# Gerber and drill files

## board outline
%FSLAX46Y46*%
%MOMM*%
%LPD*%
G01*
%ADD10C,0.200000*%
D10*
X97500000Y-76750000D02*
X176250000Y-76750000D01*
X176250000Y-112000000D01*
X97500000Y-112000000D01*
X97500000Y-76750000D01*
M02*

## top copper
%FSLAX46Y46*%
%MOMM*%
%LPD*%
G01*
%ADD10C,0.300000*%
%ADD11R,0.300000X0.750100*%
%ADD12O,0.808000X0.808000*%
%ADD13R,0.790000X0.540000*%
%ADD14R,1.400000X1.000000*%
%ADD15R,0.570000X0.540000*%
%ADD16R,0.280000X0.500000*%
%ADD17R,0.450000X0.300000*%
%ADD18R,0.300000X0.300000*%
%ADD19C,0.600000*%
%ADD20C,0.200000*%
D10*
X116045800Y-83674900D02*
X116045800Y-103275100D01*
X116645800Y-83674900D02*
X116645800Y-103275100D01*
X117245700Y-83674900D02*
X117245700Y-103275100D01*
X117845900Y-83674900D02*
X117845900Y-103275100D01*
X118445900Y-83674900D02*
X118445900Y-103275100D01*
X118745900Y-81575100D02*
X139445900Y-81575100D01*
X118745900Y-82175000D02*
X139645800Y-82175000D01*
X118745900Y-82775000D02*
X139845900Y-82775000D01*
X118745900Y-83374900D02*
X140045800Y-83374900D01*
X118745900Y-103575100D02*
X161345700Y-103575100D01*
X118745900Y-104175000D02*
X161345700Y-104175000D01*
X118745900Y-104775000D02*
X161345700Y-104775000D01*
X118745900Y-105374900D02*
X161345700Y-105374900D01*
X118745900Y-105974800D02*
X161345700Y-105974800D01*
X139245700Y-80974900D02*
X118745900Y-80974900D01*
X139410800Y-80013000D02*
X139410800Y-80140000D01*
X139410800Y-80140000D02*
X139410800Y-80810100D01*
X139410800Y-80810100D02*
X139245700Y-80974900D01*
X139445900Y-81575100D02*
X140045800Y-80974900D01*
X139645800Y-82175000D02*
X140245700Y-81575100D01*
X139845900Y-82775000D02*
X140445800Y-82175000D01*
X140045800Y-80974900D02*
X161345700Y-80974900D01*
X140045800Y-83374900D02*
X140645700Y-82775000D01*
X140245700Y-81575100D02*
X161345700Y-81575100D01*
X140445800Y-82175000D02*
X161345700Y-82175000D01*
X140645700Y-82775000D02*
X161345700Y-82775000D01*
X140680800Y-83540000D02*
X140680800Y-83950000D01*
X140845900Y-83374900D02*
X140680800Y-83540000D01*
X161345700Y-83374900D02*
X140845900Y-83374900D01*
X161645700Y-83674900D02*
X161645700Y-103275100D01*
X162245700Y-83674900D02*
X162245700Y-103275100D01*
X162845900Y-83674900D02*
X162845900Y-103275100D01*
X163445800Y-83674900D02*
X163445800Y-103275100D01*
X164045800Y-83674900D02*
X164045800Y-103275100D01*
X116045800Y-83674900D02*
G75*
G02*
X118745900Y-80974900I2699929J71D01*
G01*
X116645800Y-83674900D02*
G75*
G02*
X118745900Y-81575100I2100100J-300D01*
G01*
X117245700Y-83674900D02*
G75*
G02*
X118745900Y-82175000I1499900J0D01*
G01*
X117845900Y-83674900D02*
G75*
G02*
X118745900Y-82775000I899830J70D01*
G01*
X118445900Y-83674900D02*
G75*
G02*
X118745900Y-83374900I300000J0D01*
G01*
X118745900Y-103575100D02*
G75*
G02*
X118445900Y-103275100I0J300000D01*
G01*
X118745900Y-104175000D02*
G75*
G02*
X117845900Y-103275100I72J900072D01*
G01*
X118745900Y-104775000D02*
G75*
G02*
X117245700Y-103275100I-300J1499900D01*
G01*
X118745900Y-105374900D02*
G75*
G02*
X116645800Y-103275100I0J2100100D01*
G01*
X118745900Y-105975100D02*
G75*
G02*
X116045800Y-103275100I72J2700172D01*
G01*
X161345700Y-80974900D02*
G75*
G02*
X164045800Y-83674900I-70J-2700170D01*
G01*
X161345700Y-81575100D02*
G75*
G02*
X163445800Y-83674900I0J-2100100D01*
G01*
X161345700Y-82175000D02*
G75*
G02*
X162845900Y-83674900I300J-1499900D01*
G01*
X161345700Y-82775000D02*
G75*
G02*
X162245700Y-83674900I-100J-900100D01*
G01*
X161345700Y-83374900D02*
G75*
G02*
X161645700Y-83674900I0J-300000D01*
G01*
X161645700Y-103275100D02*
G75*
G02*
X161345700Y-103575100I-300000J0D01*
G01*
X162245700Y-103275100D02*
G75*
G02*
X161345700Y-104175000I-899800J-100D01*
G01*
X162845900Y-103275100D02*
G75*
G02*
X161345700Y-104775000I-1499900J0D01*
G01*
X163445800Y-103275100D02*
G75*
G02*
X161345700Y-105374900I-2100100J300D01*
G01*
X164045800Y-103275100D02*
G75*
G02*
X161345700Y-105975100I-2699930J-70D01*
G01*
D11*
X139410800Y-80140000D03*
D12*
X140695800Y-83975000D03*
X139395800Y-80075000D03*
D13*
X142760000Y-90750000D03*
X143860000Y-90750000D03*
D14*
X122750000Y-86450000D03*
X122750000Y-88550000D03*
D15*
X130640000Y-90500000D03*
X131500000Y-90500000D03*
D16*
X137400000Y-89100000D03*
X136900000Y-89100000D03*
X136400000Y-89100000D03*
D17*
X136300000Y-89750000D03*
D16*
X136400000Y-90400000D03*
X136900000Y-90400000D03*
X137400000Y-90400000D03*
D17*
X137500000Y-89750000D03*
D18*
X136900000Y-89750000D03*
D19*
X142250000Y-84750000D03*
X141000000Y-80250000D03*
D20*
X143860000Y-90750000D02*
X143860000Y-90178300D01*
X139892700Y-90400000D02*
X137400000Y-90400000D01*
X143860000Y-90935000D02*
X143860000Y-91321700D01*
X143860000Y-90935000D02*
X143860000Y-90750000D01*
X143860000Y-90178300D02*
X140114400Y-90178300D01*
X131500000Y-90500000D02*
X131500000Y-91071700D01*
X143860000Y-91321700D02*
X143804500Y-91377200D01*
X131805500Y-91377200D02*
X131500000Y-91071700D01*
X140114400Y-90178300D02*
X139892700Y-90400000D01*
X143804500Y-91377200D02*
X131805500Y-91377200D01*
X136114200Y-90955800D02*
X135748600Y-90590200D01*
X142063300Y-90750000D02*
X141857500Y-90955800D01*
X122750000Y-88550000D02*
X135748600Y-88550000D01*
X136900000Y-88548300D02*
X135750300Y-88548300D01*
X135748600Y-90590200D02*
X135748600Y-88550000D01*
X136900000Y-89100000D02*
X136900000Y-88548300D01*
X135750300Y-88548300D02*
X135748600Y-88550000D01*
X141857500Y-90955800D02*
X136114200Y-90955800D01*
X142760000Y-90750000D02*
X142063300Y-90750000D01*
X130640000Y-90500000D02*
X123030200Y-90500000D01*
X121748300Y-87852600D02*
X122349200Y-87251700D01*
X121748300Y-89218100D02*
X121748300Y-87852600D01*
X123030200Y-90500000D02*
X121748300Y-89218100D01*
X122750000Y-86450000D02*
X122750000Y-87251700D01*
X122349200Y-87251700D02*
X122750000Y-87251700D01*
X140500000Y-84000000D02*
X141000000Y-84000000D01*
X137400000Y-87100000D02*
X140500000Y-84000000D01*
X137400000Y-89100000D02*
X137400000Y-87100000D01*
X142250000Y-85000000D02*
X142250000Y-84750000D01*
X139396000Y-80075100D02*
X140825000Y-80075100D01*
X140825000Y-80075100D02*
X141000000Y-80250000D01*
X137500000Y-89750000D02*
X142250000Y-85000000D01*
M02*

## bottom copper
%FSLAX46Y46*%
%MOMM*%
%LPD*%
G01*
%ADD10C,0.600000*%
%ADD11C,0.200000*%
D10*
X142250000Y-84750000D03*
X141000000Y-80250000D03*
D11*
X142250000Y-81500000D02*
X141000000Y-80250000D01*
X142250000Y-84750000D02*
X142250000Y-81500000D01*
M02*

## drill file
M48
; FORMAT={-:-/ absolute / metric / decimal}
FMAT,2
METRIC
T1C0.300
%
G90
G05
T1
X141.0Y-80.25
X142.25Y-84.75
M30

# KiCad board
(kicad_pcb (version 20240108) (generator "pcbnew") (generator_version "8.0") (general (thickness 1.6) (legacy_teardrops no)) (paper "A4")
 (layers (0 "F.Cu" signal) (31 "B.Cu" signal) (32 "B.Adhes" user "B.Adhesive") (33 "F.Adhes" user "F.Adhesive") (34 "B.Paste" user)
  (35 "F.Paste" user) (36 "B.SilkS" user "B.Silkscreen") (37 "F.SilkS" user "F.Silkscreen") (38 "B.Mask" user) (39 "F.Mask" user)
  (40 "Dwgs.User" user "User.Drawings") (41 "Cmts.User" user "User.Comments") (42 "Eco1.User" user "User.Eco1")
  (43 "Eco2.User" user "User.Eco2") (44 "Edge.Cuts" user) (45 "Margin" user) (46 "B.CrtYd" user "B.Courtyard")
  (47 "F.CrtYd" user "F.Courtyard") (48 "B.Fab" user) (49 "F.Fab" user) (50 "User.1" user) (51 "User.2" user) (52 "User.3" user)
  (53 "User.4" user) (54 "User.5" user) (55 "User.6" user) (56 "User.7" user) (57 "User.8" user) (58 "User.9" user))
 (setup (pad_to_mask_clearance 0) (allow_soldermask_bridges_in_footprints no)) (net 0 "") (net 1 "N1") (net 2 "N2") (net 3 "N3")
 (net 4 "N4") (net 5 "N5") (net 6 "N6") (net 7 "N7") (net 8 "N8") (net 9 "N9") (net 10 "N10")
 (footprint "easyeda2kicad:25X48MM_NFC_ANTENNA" (layer "F.Cu") (at 140.0458 93.475)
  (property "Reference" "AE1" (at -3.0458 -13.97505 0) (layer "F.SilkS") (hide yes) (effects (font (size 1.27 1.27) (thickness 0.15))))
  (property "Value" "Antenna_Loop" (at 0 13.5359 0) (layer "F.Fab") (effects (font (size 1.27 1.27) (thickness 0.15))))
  (fp_line (start -24 -9.8001) (end -24 9.8001) (stroke (width 0.3) (type default)) (layer "F.Cu"))
  (fp_line (start -23.4 -9.8001) (end -23.4 9.8001) (stroke (width 0.3) (type default)) (layer "F.Cu"))
  (fp_line (start -22.8001 -9.8001) (end -22.8001 9.8001) (stroke (width 0.3) (type default)) (layer "F.Cu"))
  (fp_line (start -22.1999 -9.8001) (end -22.1999 9.8001) (stroke (width 0.3) (type default)) (layer "F.Cu"))
  (fp_line (start -21.5999 -9.8001) (end -21.5999 9.8001) (stroke (width 0.3) (type default)) (layer "F.Cu"))
  (fp_line (start -21.2999 -11.8999) (end -0.5999 -11.8999) (stroke (width 0.3) (type default)) (layer "F.Cu"))
  (fp_line (start -21.2999 -11.3) (end -0.4 -11.3) (stroke (width 0.3) (type default)) (layer "F.Cu"))
  (fp_line (start -21.2999 -10.7) (end -0.1999 -10.7) (stroke (width 0.3) (type default)) (layer "F.Cu"))
  (fp_line (start -21.2999 -10.1001) (end 0 -10.1001) (stroke (width 0.3) (type default)) (layer "F.Cu"))
  (fp_line (start -21.2999 10.1001) (end 21.2999 10.1001) (stroke (width 0.3) (type default)) (layer "F.Cu"))
  (fp_line (start -21.2999 10.7) (end 21.2999 10.7) (stroke (width 0.3) (type default)) (layer "F.Cu"))
  (fp_line (start -21.2999 11.3) (end 21.2999 11.3) (stroke (width 0.3) (type default)) (layer "F.Cu"))
  (fp_line (start -21.2999 11.8999) (end 21.2999 11.8999) (stroke (width 0.3) (type default)) (layer "F.Cu"))
  (fp_line (start -21.2999 12.4998) (end 21.2999 12.4998) (stroke (width 0.3) (type default)) (layer "F.Cu"))
  (fp_line (start -0.8001 -12.5001) (end -21.2999 -12.5001) (stroke (width 0.3) (type default)) (layer "F.Cu"))
  (fp_line (start -0.635 -13.462) (end -0.635 -13.335) (stroke (width 0.3) (type default)) (layer "F.Cu"))
  (fp_line (start -0.635 -13.335) (end -0.635 -12.6649) (stroke (width 0.3) (type default)) (layer "F.Cu"))
  (fp_line (start -0.635 -12.6649) (end -0.8001 -12.5001) (stroke (width 0.3) (type default)) (layer "F.Cu"))
  (fp_line (start -0.5999 -11.8999) (end 0 -12.5001) (stroke (width 0.3) (type default)) (layer "F.Cu"))
  (fp_line (start -0.4 -11.3) (end 0.1999 -11.8999) (stroke (width 0.3) (type default)) (layer "F.Cu"))
  (fp_line (start -0.1999 -10.7) (end 0.4 -11.3) (stroke (width 0.3) (type default)) (layer "F.Cu"))
  (fp_line (start 0 -12.5001) (end 21.2999 -12.5001) (stroke (width 0.3) (type default)) (layer "F.Cu"))
  (fp_line (start 0 -10.1001) (end 0.5999 -10.7) (stroke (width 0.3) (type default)) (layer "F.Cu"))
  (fp_line (start 0.1999 -11.8999) (end 21.2999 -11.8999) (stroke (width 0.3) (type default)) (layer "F.Cu"))
  (fp_line (start 0.4 -11.3) (end 21.2999 -11.3) (stroke (width 0.3) (type default)) (layer "F.Cu"))
  (fp_line (start 0.5999 -10.7) (end 21.2999 -10.7) (stroke (width 0.3) (type default)) (layer "F.Cu"))
  (fp_line (start 0.635 -9.935) (end 0.635 -9.525) (stroke (width 0.3) (type default)) (layer "F.Cu"))
  (fp_line (start 0.8001 -10.1001) (end 0.635 -9.935) (stroke (width 0.3) (type default)) (layer "F.Cu"))
  (fp_line (start 21.2999 -10.1001) (end 0.8001 -10.1001) (stroke (width 0.3) (type default)) (layer "F.Cu"))
  (fp_line (start 21.5999 -9.8001) (end 21.5999 9.8001) (stroke (width 0.3) (type default)) (layer "F.Cu"))
  (fp_line (start 22.1999 -9.8001) (end 22.1999 9.8001) (stroke (width 0.3) (type default)) (layer "F.Cu"))
  (fp_line (start 22.8001 -9.8001) (end 22.8001 9.8001) (stroke (width 0.3) (type default)) (layer "F.Cu"))
  (fp_line (start 23.4 -9.8001) (end 23.4 9.8001) (stroke (width 0.3) (type default)) (layer "F.Cu"))
  (fp_line (start 24 -9.8001) (end 24 9.8001) (stroke (width 0.3) (type default)) (layer "F.Cu"))
  (fp_arc (start -24 -9.8001) (mid -23.209174 -11.709344) (end -21.2999 -12.5001) (stroke (width 0.3) (type default)) (layer "F.Cu"))
  (fp_arc (start -23.4 -9.8001) (mid -22.784789 -11.284901) (end -21.2999 -11.8999) (stroke (width 0.3) (type default)) (layer "F.Cu"))
  (fp_arc (start -22.8001 -9.8001) (mid -22.360683 -10.860796) (end -21.2999 -11.3) (stroke (width 0.3) (type default)) (layer "F.Cu"))
  (fp_arc (start -22.1999 -9.8001) (mid -21.936311 -10.436481) (end -21.2999 -10.7) (stroke (width 0.3) (type default)) (layer "F.Cu"))
  (fp_arc (start -21.5999 -9.8001) (mid -21.512032 -10.012232) (end -21.2999 -10.1001) (stroke (width 0.3) (type default)) (layer "F.Cu"))
  (fp_arc (start -21.2999 10.1001) (mid -21.512032 10.012232) (end -21.5999 9.8001) (stroke (width 0.3) (type default)) (layer "F.Cu"))
  (fp_arc (start -21.2999 10.7) (mid -21.93624 10.43641) (end -22.1999 9.8001) (stroke (width 0.3) (type default)) (layer "F.Cu"))
  (fp_arc (start -21.2999 11.3) (mid -22.360683 10.860796) (end -22.8001 9.8001) (stroke (width 0.3) (type default)) (layer "F.Cu"))
  (fp_arc (start -21.2999 11.8999) (mid -22.784789 11.284901) (end -23.4 9.8001) (stroke (width 0.3) (type default)) (layer "F.Cu"))
  (fp_arc (start -21.2999 12.5001) (mid -23.209103 11.709273) (end -24 9.8001) (stroke (width 0.3) (type default)) (layer "F.Cu"))
  (fp_arc (start 21.2999 -12.5001) (mid 23.209103 -11.709274) (end 24 -9.8001) (stroke (width 0.3) (type default)) (layer "F.Cu"))
  (fp_arc (start 21.2999 -11.8999) (mid 22.784789 -11.284901) (end 23.4 -9.8001) (stroke (width 0.3) (type default)) (layer "F.Cu"))
  (fp_arc (start 21.2999 -11.3) (mid 22.360683 -10.860796) (end 22.8001 -9.8001) (stroke (width 0.3) (type default)) (layer "F.Cu"))
  (fp_arc (start 21.2999 -10.7) (mid 21.936231 -10.436402) (end 22.1999 -9.8001) (stroke (width 0.3) (type default)) (layer "F.Cu"))
  (fp_arc (start 21.2999 -10.1001) (mid 21.512032 -10.012232) (end 21.5999 -9.8001) (stroke (width 0.3) (type default)) (layer "F.Cu"))
  (fp_arc (start 21.5999 9.8001) (mid 21.512032 10.012232) (end 21.2999 10.1001) (stroke (width 0.3) (type default)) (layer "F.Cu"))
  (fp_arc (start 22.1999 9.8001) (mid 21.936319 10.43649) (end 21.2999 10.7) (stroke (width 0.3) (type default)) (layer "F.Cu"))
  (fp_arc (start 22.8001 9.8001) (mid 22.360683 10.860796) (end 21.2999 11.3) (stroke (width 0.3) (type default)) (layer "F.Cu"))
  (fp_arc (start 23.4 9.8001) (mid 22.784789 11.284901) (end 21.2999 11.8999) (stroke (width 0.3) (type default)) (layer "F.Cu"))
  (fp_arc (start 24 9.8001) (mid 23.209173 11.709344) (end 21.2999 12.5001) (stroke (width 0.3) (type default)) (layer "F.Cu"))
  (pad "P$1" smd rect (at -0.635 -13.335 90) (size 0.7501 0.3) (layers "F.Cu" "F.Paste" "F.Mask") (solder_mask_margin 0.1016)
   (thermal_bridge_angle 0))
  (pad "P$2" smd oval (at 0.65 -9.5) (size 0.808 0.808) (layers "F.Cu" "F.Paste" "F.Mask") (solder_mask_margin 0.1016)
   (thermal_bridge_angle 0))
  (pad "P$4" smd oval (at -0.65 -13.4) (size 0.808 0.808) (layers "F.Cu" "F.Paste" "F.Mask") (solder_mask_margin 0.1016)
   (thermal_bridge_angle 0)))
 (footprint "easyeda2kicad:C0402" (layer "F.Cu") (at 143.31 90.75)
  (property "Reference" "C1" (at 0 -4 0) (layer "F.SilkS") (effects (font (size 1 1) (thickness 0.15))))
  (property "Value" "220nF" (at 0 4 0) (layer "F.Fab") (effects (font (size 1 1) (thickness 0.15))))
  (pad "1" smd rect (at -0.55 0) (size 0.79 0.54) (layers "F.Cu" "F.Paste" "F.Mask") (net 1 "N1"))
  (pad "2" smd rect (at 0.55 0) (size 0.79 0.54) (layers "F.Cu" "F.Paste" "F.Mask") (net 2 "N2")))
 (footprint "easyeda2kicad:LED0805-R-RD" (layer "F.Cu") (at 122.75 87.5 90)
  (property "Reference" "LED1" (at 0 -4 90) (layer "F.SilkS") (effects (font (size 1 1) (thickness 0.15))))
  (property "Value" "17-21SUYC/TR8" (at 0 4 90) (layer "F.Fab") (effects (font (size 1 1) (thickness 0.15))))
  (pad "1" smd rect (at 1.05 0 270) (size 1 1.4) (layers "F.Cu" "F.Paste" "F.Mask") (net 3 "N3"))
  (pad "2" smd rect (at -1.05 0 270) (size 1 1.4) (layers "F.Cu" "F.Paste" "F.Mask") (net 1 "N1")))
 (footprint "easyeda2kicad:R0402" (layer "F.Cu") (at 131.07 90.5)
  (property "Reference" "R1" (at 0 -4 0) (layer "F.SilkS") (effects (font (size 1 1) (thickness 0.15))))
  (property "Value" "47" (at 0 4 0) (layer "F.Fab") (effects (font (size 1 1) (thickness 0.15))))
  (pad "1" smd rect (at -0.43 0) (size 0.57 0.54) (layers "F.Cu" "F.Paste" "F.Mask") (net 3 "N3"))
  (pad "2" smd rect (at 0.43 0) (size 0.57 0.54) (layers "F.Cu" "F.Paste" "F.Mask") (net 2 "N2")))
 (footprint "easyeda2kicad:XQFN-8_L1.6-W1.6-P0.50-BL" (layer "F.Cu") (at 136.9 89.75 180)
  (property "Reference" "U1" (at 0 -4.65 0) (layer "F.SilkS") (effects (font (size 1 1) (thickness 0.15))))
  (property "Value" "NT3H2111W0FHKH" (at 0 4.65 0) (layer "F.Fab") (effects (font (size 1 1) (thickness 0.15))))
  (pad "1" smd rect (at -0.5 0.65 270) (size 0.5 0.28) (layers "F.Cu" "F.Paste" "F.Mask") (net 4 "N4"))
  (pad "2" smd rect (at 0 0.65 270) (size 0.5 0.28) (layers "F.Cu" "F.Paste" "F.Mask") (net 1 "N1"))
  (pad "3" smd rect (at 0.5 0.65 270) (size 0.5 0.28) (layers "F.Cu" "F.Paste" "F.Mask") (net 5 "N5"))
  (pad "4" smd rect (at 0.6 0) (size 0.45 0.3) (layers "F.Cu" "F.Paste" "F.Mask") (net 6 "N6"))
  (pad "5" smd rect (at 0.5 -0.65 270) (size 0.5 0.28) (layers "F.Cu" "F.Paste" "F.Mask") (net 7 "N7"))
  (pad "6" smd rect (at 0 -0.65 270) (size 0.5 0.28) (layers "F.Cu" "F.Paste" "F.Mask") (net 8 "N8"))
  (pad "7" smd rect (at -0.5 -0.65 270) (size 0.5 0.28) (layers "F.Cu" "F.Paste" "F.Mask") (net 2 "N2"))
  (pad "8" smd rect (at -0.6 0) (size 0.45 0.3) (layers "F.Cu" "F.Paste" "F.Mask") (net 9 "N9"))
  (pad "9" smd rect (at 0 0) (size 0.3 0.3) (layers "F.Cu" "F.Paste" "F.Mask") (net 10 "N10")))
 (gr_rect (start 97.5 76.75) (end 176.25 112) (stroke (width 0.2) (type default)) (fill none) (layer "Edge.Cuts"))
 (segment (start 143.86 90.75) (end 143.86 90.1783) (width 0.2) (layer "F.Cu") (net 2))
 (segment (start 139.8927 90.4) (end 137.4 90.4) (width 0.2) (layer "F.Cu") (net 2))
 (segment (start 143.86 90.935) (end 143.86 91.3217) (width 0.2) (layer "F.Cu") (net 2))
 (segment (start 143.86 90.935) (end 143.86 90.75) (width 0.2) (layer "F.Cu") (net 2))
 (segment (start 143.86 90.1783) (end 140.1144 90.1783) (width 0.2) (layer "F.Cu") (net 2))
 (segment (start 131.5 90.5) (end 131.5 91.0717) (width 0.2) (layer "F.Cu") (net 2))
 (segment (start 143.86 91.3217) (end 143.8045 91.3772) (width 0.2) (layer "F.Cu") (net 2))
 (segment (start 131.8055 91.3772) (end 131.5 91.0717) (width 0.2) (layer "F.Cu") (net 2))
 (segment (start 140.1144 90.1783) (end 139.8927 90.4) (width 0.2) (layer "F.Cu") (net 2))
 (segment (start 143.8045 91.3772) (end 131.8055 91.3772) (width 0.2) (layer "F.Cu") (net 2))
 (segment (start 136.1142 90.9558) (end 135.7486 90.5902) (width 0.2) (layer "F.Cu") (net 1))
 (segment (start 142.0633 90.75) (end 141.8575 90.9558) (width 0.2) (layer "F.Cu") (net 1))
 (segment (start 122.75 88.55) (end 135.7486 88.55) (width 0.2) (layer "F.Cu") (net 1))
 (segment (start 136.9 88.5483) (end 135.7503 88.5483) (width 0.2) (layer "F.Cu") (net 1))
 (segment (start 135.7486 90.5902) (end 135.7486 88.55) (width 0.2) (layer "F.Cu") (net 1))
 (segment (start 136.9 89.1) (end 136.9 88.5483) (width 0.2) (layer "F.Cu") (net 1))
 (segment (start 135.7503 88.5483) (end 135.7486 88.55) (width 0.2) (layer "F.Cu") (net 1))
 (segment (start 141.8575 90.9558) (end 136.1142 90.9558) (width 0.2) (layer "F.Cu") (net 1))
 (segment (start 142.76 90.75) (end 142.0633 90.75) (width 0.2) (layer "F.Cu") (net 1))
 (segment (start 130.64 90.5) (end 123.0302 90.5) (width 0.2) (layer "F.Cu") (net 3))
 (segment (start 121.7483 87.8526) (end 122.3492 87.2517) (width 0.2) (layer "F.Cu") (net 3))
 (segment (start 121.7483 89.2181) (end 121.7483 87.8526) (width 0.2) (layer "F.Cu") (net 3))
 (segment (start 123.0302 90.5) (end 121.7483 89.2181) (width 0.2) (layer "F.Cu") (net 3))
 (segment (start 122.75 86.45) (end 122.75 87.2517) (width 0.2) (layer "F.Cu") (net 3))
 (segment (start 122.3492 87.2517) (end 122.75 87.2517) (width 0.2) (layer "F.Cu") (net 3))
 (segment (start 140.5 84) (end 141 84) (width 0.2) (layer "F.Cu") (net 4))
 (segment (start 137.4 87.1) (end 140.5 84) (width 0.2) (layer "F.Cu") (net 4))
 (segment (start 137.4 89.1) (end 137.4 87.1) (width 0.2) (layer "F.Cu") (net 4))
 (segment (start 142.25 85) (end 142.25 84.75) (width 0.2) (layer "F.Cu") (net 9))
 (segment (start 139.396 80.0751) (end 140.825 80.0751) (width 0.2) (layer "F.Cu") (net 9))
 (segment (start 140.825 80.0751) (end 141 80.25) (width 0.2) (layer "F.Cu") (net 9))
 (segment (start 137.5 89.75) (end 142.25 85) (width 0.2) (layer "F.Cu") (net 9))
 (via (at 142.25 84.75) (size 0.6) (drill 0.3) (layers "F.Cu" "B.Cu") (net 9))
 (via (at 141 80.25) (size 0.6) (drill 0.3) (layers "F.Cu" "B.Cu") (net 9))
 (segment (start 142.25 81.5) (end 141 80.25) (width 0.2) (layer "B.Cu") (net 9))
 (segment (start 142.25 84.75) (end 142.25 81.5) (width 0.2) (layer "B.Cu") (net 9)))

